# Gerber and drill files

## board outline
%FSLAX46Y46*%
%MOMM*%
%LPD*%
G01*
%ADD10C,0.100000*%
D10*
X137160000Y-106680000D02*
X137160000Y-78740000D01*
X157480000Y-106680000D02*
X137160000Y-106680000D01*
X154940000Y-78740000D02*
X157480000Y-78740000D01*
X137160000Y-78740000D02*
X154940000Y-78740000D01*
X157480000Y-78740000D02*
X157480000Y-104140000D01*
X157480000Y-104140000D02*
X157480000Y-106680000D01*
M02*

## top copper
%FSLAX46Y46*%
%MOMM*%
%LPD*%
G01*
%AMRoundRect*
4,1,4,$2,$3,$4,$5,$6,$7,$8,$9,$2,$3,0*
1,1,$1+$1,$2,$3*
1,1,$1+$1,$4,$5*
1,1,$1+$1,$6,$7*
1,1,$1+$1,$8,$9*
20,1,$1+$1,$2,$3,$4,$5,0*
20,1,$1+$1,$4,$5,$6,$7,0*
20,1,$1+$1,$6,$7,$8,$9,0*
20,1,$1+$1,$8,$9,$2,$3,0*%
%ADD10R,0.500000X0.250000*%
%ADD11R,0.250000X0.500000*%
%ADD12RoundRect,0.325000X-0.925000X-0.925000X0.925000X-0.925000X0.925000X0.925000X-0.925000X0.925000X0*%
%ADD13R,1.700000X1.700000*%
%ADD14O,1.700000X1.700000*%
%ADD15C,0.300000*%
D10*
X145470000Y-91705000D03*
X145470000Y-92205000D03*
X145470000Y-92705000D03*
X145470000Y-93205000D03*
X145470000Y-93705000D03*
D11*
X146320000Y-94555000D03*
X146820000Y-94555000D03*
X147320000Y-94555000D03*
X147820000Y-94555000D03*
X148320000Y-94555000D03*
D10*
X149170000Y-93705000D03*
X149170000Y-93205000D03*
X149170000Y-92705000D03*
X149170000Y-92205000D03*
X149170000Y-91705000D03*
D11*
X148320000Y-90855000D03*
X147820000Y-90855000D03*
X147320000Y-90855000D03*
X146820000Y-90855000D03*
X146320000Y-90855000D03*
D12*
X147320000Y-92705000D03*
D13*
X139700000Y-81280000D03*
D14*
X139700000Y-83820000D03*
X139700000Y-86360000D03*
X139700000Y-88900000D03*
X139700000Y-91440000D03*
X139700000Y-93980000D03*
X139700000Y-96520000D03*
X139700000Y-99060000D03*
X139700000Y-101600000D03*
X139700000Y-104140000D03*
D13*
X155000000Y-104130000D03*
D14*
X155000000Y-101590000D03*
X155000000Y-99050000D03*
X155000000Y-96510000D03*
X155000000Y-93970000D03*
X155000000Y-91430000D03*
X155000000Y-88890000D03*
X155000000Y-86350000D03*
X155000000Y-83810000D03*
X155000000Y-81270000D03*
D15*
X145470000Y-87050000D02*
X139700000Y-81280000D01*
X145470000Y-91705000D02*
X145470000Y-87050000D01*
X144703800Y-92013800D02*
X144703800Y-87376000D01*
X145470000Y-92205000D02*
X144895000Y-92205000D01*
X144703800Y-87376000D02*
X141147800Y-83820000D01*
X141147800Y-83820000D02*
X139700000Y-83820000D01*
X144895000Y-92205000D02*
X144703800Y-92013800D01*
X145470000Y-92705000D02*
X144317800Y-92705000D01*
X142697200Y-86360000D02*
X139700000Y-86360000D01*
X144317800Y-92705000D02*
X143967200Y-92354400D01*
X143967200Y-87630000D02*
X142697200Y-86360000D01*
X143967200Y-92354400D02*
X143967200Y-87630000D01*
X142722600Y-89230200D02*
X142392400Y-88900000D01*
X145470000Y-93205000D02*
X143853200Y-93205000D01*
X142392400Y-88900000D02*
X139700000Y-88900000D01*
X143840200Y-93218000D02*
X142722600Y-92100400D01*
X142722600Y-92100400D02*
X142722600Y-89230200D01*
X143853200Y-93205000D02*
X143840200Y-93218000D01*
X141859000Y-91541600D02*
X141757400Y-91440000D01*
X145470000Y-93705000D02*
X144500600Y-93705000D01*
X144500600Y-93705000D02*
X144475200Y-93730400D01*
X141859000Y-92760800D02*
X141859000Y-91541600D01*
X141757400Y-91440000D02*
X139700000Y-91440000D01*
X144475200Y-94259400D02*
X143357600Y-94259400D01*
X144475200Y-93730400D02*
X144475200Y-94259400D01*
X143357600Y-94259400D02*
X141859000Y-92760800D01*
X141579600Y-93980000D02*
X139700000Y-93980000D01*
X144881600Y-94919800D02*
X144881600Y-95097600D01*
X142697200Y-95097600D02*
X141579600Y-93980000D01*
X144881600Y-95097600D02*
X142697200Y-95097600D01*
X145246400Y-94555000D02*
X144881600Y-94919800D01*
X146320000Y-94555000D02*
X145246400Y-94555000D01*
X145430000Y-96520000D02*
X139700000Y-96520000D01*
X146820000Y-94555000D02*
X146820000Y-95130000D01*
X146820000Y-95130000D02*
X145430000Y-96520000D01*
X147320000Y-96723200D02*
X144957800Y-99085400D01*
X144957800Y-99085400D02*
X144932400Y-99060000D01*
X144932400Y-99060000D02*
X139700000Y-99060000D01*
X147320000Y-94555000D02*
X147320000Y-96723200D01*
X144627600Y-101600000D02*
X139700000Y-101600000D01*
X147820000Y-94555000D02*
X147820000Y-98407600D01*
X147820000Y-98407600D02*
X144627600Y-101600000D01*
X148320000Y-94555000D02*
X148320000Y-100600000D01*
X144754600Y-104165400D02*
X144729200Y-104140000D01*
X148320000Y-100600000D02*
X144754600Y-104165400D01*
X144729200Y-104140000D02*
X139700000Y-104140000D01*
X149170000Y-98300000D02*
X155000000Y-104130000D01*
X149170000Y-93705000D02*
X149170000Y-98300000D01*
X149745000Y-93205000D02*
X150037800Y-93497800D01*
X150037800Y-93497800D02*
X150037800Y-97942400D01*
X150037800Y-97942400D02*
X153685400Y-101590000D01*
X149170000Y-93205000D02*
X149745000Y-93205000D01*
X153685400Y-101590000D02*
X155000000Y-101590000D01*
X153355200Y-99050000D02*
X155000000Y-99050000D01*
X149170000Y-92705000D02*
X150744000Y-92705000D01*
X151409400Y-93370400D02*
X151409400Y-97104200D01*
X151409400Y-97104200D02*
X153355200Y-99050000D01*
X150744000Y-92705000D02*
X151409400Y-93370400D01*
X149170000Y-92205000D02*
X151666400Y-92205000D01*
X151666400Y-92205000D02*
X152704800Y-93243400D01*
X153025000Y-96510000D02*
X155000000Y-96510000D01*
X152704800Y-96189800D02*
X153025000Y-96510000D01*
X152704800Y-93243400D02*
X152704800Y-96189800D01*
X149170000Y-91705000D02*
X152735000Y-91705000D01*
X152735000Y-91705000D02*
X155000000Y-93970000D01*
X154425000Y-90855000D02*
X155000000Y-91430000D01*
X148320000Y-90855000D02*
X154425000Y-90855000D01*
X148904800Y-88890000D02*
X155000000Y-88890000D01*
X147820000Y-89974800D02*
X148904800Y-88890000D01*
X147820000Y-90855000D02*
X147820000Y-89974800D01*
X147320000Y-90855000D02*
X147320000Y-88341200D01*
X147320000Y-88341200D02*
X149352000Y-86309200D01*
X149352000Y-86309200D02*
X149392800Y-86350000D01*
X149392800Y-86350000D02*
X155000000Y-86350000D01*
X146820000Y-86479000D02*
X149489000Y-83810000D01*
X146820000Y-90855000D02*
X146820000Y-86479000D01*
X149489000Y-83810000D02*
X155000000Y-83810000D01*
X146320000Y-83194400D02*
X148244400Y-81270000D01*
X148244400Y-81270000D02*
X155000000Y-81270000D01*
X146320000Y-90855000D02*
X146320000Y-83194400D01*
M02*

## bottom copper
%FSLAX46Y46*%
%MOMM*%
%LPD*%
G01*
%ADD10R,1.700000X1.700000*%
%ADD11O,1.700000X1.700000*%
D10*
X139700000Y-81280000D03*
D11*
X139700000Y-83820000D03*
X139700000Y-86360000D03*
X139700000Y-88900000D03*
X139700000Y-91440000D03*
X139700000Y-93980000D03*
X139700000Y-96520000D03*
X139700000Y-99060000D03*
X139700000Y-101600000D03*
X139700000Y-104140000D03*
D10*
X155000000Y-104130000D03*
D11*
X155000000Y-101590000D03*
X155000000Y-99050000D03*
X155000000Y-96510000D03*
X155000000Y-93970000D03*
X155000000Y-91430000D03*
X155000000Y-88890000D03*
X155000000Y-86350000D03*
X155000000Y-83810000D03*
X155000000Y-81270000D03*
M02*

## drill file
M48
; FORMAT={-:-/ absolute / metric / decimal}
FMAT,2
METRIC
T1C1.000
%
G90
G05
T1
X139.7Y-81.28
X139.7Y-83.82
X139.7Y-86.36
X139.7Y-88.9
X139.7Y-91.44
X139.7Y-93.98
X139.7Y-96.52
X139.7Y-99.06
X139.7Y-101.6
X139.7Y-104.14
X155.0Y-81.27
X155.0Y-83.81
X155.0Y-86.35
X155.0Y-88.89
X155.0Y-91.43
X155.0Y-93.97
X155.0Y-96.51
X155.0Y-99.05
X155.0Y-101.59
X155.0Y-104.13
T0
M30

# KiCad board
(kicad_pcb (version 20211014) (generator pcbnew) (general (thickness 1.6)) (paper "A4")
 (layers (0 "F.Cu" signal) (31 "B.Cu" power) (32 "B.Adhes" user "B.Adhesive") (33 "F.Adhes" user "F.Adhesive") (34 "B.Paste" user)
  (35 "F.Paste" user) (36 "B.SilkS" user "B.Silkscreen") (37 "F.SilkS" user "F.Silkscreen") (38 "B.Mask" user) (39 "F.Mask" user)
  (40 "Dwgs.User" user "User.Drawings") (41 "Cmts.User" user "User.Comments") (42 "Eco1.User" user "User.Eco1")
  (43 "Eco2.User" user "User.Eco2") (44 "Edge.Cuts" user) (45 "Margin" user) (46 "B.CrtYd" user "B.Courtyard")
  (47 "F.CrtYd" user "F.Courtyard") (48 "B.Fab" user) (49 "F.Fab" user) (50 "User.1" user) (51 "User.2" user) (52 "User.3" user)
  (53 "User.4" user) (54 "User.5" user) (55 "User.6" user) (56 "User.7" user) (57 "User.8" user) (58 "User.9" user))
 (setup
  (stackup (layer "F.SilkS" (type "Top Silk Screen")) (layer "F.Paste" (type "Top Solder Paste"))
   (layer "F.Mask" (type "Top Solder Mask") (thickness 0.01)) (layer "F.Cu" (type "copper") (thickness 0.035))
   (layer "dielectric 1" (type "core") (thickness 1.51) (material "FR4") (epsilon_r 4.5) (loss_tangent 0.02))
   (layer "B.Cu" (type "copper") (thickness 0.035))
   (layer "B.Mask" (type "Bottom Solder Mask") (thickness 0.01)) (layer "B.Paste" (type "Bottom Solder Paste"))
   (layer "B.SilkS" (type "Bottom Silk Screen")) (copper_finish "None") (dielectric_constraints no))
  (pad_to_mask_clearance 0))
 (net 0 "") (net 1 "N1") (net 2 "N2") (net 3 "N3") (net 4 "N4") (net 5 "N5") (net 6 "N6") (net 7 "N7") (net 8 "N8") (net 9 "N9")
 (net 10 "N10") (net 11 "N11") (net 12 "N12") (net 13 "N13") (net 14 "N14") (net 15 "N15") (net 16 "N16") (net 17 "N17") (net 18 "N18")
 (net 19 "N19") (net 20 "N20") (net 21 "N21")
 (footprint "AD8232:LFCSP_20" (layer "F.Cu") (at 147.32 92.705)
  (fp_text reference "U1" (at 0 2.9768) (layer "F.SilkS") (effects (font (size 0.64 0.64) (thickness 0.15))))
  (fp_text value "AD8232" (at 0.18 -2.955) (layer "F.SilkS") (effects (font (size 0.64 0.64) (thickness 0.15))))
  (pad "1" smd rect locked (at -1.85 -1 270) (size 0.25 0.5) (layers "F.Cu" "F.Paste" "F.Mask") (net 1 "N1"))
  (pad "2" smd rect locked (at -1.85 -0.5 270) (size 0.25 0.5) (layers "F.Cu" "F.Paste" "F.Mask") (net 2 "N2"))
  (pad "3" smd rect locked (at -1.85 0 270) (size 0.25 0.5) (layers "F.Cu" "F.Paste" "F.Mask") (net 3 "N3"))
  (pad "4" smd rect locked (at -1.85 0.5 270) (size 0.25 0.5) (layers "F.Cu" "F.Paste" "F.Mask") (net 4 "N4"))
  (pad "5" smd rect locked (at -1.85 1 270) (size 0.25 0.5) (layers "F.Cu" "F.Paste" "F.Mask") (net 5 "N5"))
  (pad "6" smd rect locked (at -1 1.85) (size 0.25 0.5) (layers "F.Cu" "F.Paste" "F.Mask") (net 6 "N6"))
  (pad "7" smd rect locked (at -0.5 1.85) (size 0.25 0.5) (layers "F.Cu" "F.Paste" "F.Mask") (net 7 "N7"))
  (pad "8" smd rect locked (at 0 1.85) (size 0.25 0.5) (layers "F.Cu" "F.Paste" "F.Mask") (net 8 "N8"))
  (pad "9" smd rect locked (at 0.5 1.85) (size 0.25 0.5) (layers "F.Cu" "F.Paste" "F.Mask") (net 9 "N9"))
  (pad "10" smd rect locked (at 1 1.85) (size 0.25 0.5) (layers "F.Cu" "F.Paste" "F.Mask") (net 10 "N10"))
  (pad "11" smd rect locked (at 1.85 1 90) (size 0.25 0.5) (layers "F.Cu" "F.Paste" "F.Mask") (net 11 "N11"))
  (pad "12" smd rect locked (at 1.85 0.5 90) (size 0.25 0.5) (layers "F.Cu" "F.Paste" "F.Mask") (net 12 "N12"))
  (pad "13" smd rect locked (at 1.85 0 90) (size 0.25 0.5) (layers "F.Cu" "F.Paste" "F.Mask") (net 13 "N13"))
  (pad "14" smd rect locked (at 1.85 -0.5 90) (size 0.25 0.5) (layers "F.Cu" "F.Paste" "F.Mask") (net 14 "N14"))
  (pad "15" smd rect locked (at 1.85 -1 90) (size 0.25 0.5) (layers "F.Cu" "F.Paste" "F.Mask") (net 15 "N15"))
  (pad "16" smd rect locked (at 1 -1.85 180) (size 0.25 0.5) (layers "F.Cu" "F.Paste" "F.Mask") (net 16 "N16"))
  (pad "17" smd rect locked (at 0.5 -1.85 180) (size 0.25 0.5) (layers "F.Cu" "F.Paste" "F.Mask") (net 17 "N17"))
  (pad "18" smd rect locked (at 0 -1.85 180) (size 0.25 0.5) (layers "F.Cu" "F.Paste" "F.Mask") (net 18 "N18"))
  (pad "19" smd rect locked (at -0.5 -1.85 180) (size 0.25 0.5) (layers "F.Cu" "F.Paste" "F.Mask") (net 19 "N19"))
  (pad "20" smd rect locked (at -1 -1.85 180) (size 0.25 0.5) (layers "F.Cu" "F.Paste" "F.Mask") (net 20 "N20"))
  (pad "PAD" smd roundrect locked (at 0 0) (size 2.5 2.5) (layers "F.Cu" "F.Mask") (roundrect_rratio 0.13) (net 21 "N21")))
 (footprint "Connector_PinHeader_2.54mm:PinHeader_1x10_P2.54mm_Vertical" (layer "B.Cu") (at 139.7 81.28 180)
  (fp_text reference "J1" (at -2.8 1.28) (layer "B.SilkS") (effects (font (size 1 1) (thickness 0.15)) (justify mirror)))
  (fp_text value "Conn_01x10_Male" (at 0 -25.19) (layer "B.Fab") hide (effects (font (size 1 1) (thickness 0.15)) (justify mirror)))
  (pad "1" thru_hole rect (at 0 0 180) (size 1.7 1.7) (drill 1) (layers *.Cu *.Mask) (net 1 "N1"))
  (pad "2" thru_hole oval (at 0 -2.54 180) (size 1.7 1.7) (drill 1) (layers *.Cu *.Mask) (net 2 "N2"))
  (pad "3" thru_hole oval (at 0 -5.08 180) (size 1.7 1.7) (drill 1) (layers *.Cu *.Mask) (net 3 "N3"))
  (pad "4" thru_hole oval (at 0 -7.62 180) (size 1.7 1.7) (drill 1) (layers *.Cu *.Mask) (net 4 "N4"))
  (pad "5" thru_hole oval (at 0 -10.16 180) (size 1.7 1.7) (drill 1) (layers *.Cu *.Mask) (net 5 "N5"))
  (pad "6" thru_hole oval (at 0 -12.7 180) (size 1.7 1.7) (drill 1) (layers *.Cu *.Mask) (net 6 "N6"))
  (pad "7" thru_hole oval (at 0 -15.24 180) (size 1.7 1.7) (drill 1) (layers *.Cu *.Mask) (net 7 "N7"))
  (pad "8" thru_hole oval (at 0 -17.78 180) (size 1.7 1.7) (drill 1) (layers *.Cu *.Mask) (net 8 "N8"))
  (pad "9" thru_hole oval (at 0 -20.32 180) (size 1.7 1.7) (drill 1) (layers *.Cu *.Mask) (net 9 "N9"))
  (pad "10" thru_hole oval (at 0 -22.86 180) (size 1.7 1.7) (drill 1) (layers *.Cu *.Mask) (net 10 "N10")))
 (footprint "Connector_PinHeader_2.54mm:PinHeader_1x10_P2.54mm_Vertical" (layer "B.Cu") (at 155 104.13)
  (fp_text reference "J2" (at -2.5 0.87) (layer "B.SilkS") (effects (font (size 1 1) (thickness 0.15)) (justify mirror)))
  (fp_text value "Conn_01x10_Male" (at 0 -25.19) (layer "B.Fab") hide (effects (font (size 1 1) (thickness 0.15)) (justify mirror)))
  (pad "1" thru_hole rect (at 0 0) (size 1.7 1.7) (drill 1) (layers *.Cu *.Mask) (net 11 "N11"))
  (pad "2" thru_hole oval (at 0 -2.54) (size 1.7 1.7) (drill 1) (layers *.Cu *.Mask) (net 12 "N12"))
  (pad "3" thru_hole oval (at 0 -5.08) (size 1.7 1.7) (drill 1) (layers *.Cu *.Mask) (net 13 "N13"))
  (pad "4" thru_hole oval (at 0 -7.62) (size 1.7 1.7) (drill 1) (layers *.Cu *.Mask) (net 14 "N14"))
  (pad "5" thru_hole oval (at 0 -10.16) (size 1.7 1.7) (drill 1) (layers *.Cu *.Mask) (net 15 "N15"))
  (pad "6" thru_hole oval (at 0 -12.7) (size 1.7 1.7) (drill 1) (layers *.Cu *.Mask) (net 16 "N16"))
  (pad "7" thru_hole oval (at 0 -15.24) (size 1.7 1.7) (drill 1) (layers *.Cu *.Mask) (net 17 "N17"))
  (pad "8" thru_hole oval (at 0 -17.78) (size 1.7 1.7) (drill 1) (layers *.Cu *.Mask) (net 18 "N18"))
  (pad "9" thru_hole oval (at 0 -20.32) (size 1.7 1.7) (drill 1) (layers *.Cu *.Mask) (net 19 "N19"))
  (pad "10" thru_hole oval (at 0 -22.86) (size 1.7 1.7) (drill 1) (layers *.Cu *.Mask) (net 20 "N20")))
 (gr_line (start 137.16 106.68) (end 137.16 78.74) (layer "Edge.Cuts") (width 0.1))
 (gr_line (start 157.48 106.68) (end 137.16 106.68) (layer "Edge.Cuts") (width 0.1))
 (gr_line (start 154.94 78.74) (end 157.48 78.74) (layer "Edge.Cuts") (width 0.1))
 (gr_line (start 137.16 78.74) (end 154.94 78.74) (layer "Edge.Cuts") (width 0.1))
 (gr_line (start 157.48 78.74) (end 157.48 104.14) (layer "Edge.Cuts") (width 0.1))
 (gr_line (start 157.48 104.14) (end 157.48 106.68) (layer "Edge.Cuts") (width 0.1))
 (segment (start 145.47 87.05) (end 139.7 81.28) (width 0.3) (layer "F.Cu") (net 1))
 (segment (start 145.47 91.705) (end 145.47 87.05) (width 0.3) (layer "F.Cu") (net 1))
 (segment (start 144.7038 92.0138) (end 144.7038 87.376) (width 0.3) (layer "F.Cu") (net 2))
 (segment (start 145.47 92.205) (end 144.895 92.205) (width 0.3) (layer "F.Cu") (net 2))
 (segment (start 144.7038 87.376) (end 141.1478 83.82) (width 0.3) (layer "F.Cu") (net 2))
 (segment (start 141.1478 83.82) (end 139.7 83.82) (width 0.3) (layer "F.Cu") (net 2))
 (segment (start 144.895 92.205) (end 144.7038 92.0138) (width 0.3) (layer "F.Cu") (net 2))
 (segment (start 145.47 92.705) (end 144.3178 92.705) (width 0.3) (layer "F.Cu") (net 3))
 (segment (start 142.6972 86.36) (end 139.7 86.36) (width 0.3) (layer "F.Cu") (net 3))
 (segment (start 144.3178 92.705) (end 143.9672 92.3544) (width 0.3) (layer "F.Cu") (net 3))
 (segment (start 143.9672 87.63) (end 142.6972 86.36) (width 0.3) (layer "F.Cu") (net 3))
 (segment (start 143.9672 92.3544) (end 143.9672 87.63) (width 0.3) (layer "F.Cu") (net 3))
 (segment (start 142.7226 89.2302) (end 142.3924 88.9) (width 0.3) (layer "F.Cu") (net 4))
 (segment (start 145.47 93.205) (end 143.8532 93.205) (width 0.3) (layer "F.Cu") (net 4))
 (segment (start 142.3924 88.9) (end 139.7 88.9) (width 0.3) (layer "F.Cu") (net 4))
 (segment (start 143.8402 93.218) (end 142.7226 92.1004) (width 0.3) (layer "F.Cu") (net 4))
 (segment (start 142.7226 92.1004) (end 142.7226 89.2302) (width 0.3) (layer "F.Cu") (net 4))
 (segment (start 143.8532 93.205) (end 143.8402 93.218) (width 0.3) (layer "F.Cu") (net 4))
 (segment (start 141.859 91.5416) (end 141.7574 91.44) (width 0.3) (layer "F.Cu") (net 5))
 (segment (start 145.47 93.705) (end 144.5006 93.705) (width 0.3) (layer "F.Cu") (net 5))
 (segment (start 144.5006 93.705) (end 144.4752 93.7304) (width 0.3) (layer "F.Cu") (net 5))
 (segment (start 141.859 92.7608) (end 141.859 91.5416) (width 0.3) (layer "F.Cu") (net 5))
 (segment (start 141.7574 91.44) (end 139.7 91.44) (width 0.3) (layer "F.Cu") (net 5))
 (segment (start 144.4752 94.2594) (end 143.3576 94.2594) (width 0.3) (layer "F.Cu") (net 5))
 (segment (start 144.4752 93.7304) (end 144.4752 94.2594) (width 0.3) (layer "F.Cu") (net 5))
 (segment (start 143.3576 94.2594) (end 141.859 92.7608) (width 0.3) (layer "F.Cu") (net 5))
 (segment (start 141.5796 93.98) (end 139.7 93.98) (width 0.3) (layer "F.Cu") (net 6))
 (segment (start 144.8816 94.9198) (end 144.8816 95.0976) (width 0.3) (layer "F.Cu") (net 6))
 (segment (start 142.6972 95.0976) (end 141.5796 93.98) (width 0.3) (layer "F.Cu") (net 6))
 (segment (start 144.8816 95.0976) (end 142.6972 95.0976) (width 0.3) (layer "F.Cu") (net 6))
 (segment (start 145.2464 94.555) (end 144.8816 94.9198) (width 0.3) (layer "F.Cu") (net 6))
 (segment (start 146.32 94.555) (end 145.2464 94.555) (width 0.3) (layer "F.Cu") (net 6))
 (segment (start 145.43 96.52) (end 139.7 96.52) (width 0.3) (layer "F.Cu") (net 7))
 (segment (start 146.82 94.555) (end 146.82 95.13) (width 0.3) (layer "F.Cu") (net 7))
 (segment (start 146.82 95.13) (end 145.43 96.52) (width 0.3) (layer "F.Cu") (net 7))
 (segment (start 147.32 96.7232) (end 144.9578 99.0854) (width 0.3) (layer "F.Cu") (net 8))
 (segment (start 144.9578 99.0854) (end 144.9324 99.06) (width 0.3) (layer "F.Cu") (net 8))
 (segment (start 144.9324 99.06) (end 139.7 99.06) (width 0.3) (layer "F.Cu") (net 8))
 (segment (start 147.32 94.555) (end 147.32 96.7232) (width 0.3) (layer "F.Cu") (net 8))
 (segment (start 144.6276 101.6) (end 139.7 101.6) (width 0.3) (layer "F.Cu") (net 9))
 (segment (start 147.82 94.555) (end 147.82 98.4076) (width 0.3) (layer "F.Cu") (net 9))
 (segment (start 147.82 98.4076) (end 144.6276 101.6) (width 0.3) (layer "F.Cu") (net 9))
 (segment (start 148.32 94.555) (end 148.32 100.6) (width 0.3) (layer "F.Cu") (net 10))
 (segment (start 144.7546 104.1654) (end 144.7292 104.14) (width 0.3) (layer "F.Cu") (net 10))
 (segment (start 148.32 100.6) (end 144.7546 104.1654) (width 0.3) (layer "F.Cu") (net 10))
 (segment (start 144.7292 104.14) (end 139.7 104.14) (width 0.3) (layer "F.Cu") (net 10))
 (segment (start 149.17 98.3) (end 155 104.13) (width 0.3) (layer "F.Cu") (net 11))
 (segment (start 149.17 93.705) (end 149.17 98.3) (width 0.3) (layer "F.Cu") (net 11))
 (segment (start 149.745 93.205) (end 150.0378 93.4978) (width 0.3) (layer "F.Cu") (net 12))
 (segment (start 150.0378 93.4978) (end 150.0378 97.9424) (width 0.3) (layer "F.Cu") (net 12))
 (segment (start 150.0378 97.9424) (end 153.6854 101.59) (width 0.3) (layer "F.Cu") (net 12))
 (segment (start 149.17 93.205) (end 149.745 93.205) (width 0.3) (layer "F.Cu") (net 12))
 (segment (start 153.6854 101.59) (end 155 101.59) (width 0.3) (layer "F.Cu") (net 12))
 (segment (start 153.3552 99.05) (end 155 99.05) (width 0.3) (layer "F.Cu") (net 13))
 (segment (start 149.17 92.705) (end 150.744 92.705) (width 0.3) (layer "F.Cu") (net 13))
 (segment (start 151.4094 93.3704) (end 151.4094 97.1042) (width 0.3) (layer "F.Cu") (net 13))
 (segment (start 151.4094 97.1042) (end 153.3552 99.05) (width 0.3) (layer "F.Cu") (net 13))
 (segment (start 150.744 92.705) (end 151.4094 93.3704) (width 0.3) (layer "F.Cu") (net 13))
 (segment (start 149.17 92.205) (end 151.6664 92.205) (width 0.3) (layer "F.Cu") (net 14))
 (segment (start 151.6664 92.205) (end 152.7048 93.2434) (width 0.3) (layer "F.Cu") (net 14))
 (segment (start 153.025 96.51) (end 155 96.51) (width 0.3) (layer "F.Cu") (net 14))
 (segment (start 152.7048 96.1898) (end 153.025 96.51) (width 0.3) (layer "F.Cu") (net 14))
 (segment (start 152.7048 93.2434) (end 152.7048 96.1898) (width 0.3) (layer "F.Cu") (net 14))
 (segment (start 149.17 91.705) (end 152.735 91.705) (width 0.3) (layer "F.Cu") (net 15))
 (segment (start 152.735 91.705) (end 155 93.97) (width 0.3) (layer "F.Cu") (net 15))
 (segment (start 154.425 90.855) (end 155 91.43) (width 0.3) (layer "F.Cu") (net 16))
 (segment (start 148.32 90.855) (end 154.425 90.855) (width 0.3) (layer "F.Cu") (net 16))
 (segment (start 148.9048 88.89) (end 155 88.89) (width 0.3) (layer "F.Cu") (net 17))
 (segment (start 147.82 89.9748) (end 148.9048 88.89) (width 0.3) (layer "F.Cu") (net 17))
 (segment (start 147.82 90.855) (end 147.82 89.9748) (width 0.3) (layer "F.Cu") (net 17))
 (segment (start 147.32 90.855) (end 147.32 88.3412) (width 0.3) (layer "F.Cu") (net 18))
 (segment (start 147.32 88.3412) (end 149.352 86.3092) (width 0.3) (layer "F.Cu") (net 18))
 (segment (start 149.352 86.3092) (end 149.3928 86.35) (width 0.3) (layer "F.Cu") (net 18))
 (segment (start 149.3928 86.35) (end 155 86.35) (width 0.3) (layer "F.Cu") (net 18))
 (segment (start 146.82 86.479) (end 149.489 83.81) (width 0.3) (layer "F.Cu") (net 19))
 (segment (start 146.82 90.855) (end 146.82 86.479) (width 0.3) (layer "F.Cu") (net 19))
 (segment (start 149.489 83.81) (end 155 83.81) (width 0.3) (layer "F.Cu") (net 19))
 (segment (start 146.32 83.1944) (end 148.2444 81.27) (width 0.3) (layer "F.Cu") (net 20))
 (segment (start 148.2444 81.27) (end 155 81.27) (width 0.3) (layer "F.Cu") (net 20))
 (segment (start 146.32 90.855) (end 146.32 83.1944) (width 0.3) (layer "F.Cu") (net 20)))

